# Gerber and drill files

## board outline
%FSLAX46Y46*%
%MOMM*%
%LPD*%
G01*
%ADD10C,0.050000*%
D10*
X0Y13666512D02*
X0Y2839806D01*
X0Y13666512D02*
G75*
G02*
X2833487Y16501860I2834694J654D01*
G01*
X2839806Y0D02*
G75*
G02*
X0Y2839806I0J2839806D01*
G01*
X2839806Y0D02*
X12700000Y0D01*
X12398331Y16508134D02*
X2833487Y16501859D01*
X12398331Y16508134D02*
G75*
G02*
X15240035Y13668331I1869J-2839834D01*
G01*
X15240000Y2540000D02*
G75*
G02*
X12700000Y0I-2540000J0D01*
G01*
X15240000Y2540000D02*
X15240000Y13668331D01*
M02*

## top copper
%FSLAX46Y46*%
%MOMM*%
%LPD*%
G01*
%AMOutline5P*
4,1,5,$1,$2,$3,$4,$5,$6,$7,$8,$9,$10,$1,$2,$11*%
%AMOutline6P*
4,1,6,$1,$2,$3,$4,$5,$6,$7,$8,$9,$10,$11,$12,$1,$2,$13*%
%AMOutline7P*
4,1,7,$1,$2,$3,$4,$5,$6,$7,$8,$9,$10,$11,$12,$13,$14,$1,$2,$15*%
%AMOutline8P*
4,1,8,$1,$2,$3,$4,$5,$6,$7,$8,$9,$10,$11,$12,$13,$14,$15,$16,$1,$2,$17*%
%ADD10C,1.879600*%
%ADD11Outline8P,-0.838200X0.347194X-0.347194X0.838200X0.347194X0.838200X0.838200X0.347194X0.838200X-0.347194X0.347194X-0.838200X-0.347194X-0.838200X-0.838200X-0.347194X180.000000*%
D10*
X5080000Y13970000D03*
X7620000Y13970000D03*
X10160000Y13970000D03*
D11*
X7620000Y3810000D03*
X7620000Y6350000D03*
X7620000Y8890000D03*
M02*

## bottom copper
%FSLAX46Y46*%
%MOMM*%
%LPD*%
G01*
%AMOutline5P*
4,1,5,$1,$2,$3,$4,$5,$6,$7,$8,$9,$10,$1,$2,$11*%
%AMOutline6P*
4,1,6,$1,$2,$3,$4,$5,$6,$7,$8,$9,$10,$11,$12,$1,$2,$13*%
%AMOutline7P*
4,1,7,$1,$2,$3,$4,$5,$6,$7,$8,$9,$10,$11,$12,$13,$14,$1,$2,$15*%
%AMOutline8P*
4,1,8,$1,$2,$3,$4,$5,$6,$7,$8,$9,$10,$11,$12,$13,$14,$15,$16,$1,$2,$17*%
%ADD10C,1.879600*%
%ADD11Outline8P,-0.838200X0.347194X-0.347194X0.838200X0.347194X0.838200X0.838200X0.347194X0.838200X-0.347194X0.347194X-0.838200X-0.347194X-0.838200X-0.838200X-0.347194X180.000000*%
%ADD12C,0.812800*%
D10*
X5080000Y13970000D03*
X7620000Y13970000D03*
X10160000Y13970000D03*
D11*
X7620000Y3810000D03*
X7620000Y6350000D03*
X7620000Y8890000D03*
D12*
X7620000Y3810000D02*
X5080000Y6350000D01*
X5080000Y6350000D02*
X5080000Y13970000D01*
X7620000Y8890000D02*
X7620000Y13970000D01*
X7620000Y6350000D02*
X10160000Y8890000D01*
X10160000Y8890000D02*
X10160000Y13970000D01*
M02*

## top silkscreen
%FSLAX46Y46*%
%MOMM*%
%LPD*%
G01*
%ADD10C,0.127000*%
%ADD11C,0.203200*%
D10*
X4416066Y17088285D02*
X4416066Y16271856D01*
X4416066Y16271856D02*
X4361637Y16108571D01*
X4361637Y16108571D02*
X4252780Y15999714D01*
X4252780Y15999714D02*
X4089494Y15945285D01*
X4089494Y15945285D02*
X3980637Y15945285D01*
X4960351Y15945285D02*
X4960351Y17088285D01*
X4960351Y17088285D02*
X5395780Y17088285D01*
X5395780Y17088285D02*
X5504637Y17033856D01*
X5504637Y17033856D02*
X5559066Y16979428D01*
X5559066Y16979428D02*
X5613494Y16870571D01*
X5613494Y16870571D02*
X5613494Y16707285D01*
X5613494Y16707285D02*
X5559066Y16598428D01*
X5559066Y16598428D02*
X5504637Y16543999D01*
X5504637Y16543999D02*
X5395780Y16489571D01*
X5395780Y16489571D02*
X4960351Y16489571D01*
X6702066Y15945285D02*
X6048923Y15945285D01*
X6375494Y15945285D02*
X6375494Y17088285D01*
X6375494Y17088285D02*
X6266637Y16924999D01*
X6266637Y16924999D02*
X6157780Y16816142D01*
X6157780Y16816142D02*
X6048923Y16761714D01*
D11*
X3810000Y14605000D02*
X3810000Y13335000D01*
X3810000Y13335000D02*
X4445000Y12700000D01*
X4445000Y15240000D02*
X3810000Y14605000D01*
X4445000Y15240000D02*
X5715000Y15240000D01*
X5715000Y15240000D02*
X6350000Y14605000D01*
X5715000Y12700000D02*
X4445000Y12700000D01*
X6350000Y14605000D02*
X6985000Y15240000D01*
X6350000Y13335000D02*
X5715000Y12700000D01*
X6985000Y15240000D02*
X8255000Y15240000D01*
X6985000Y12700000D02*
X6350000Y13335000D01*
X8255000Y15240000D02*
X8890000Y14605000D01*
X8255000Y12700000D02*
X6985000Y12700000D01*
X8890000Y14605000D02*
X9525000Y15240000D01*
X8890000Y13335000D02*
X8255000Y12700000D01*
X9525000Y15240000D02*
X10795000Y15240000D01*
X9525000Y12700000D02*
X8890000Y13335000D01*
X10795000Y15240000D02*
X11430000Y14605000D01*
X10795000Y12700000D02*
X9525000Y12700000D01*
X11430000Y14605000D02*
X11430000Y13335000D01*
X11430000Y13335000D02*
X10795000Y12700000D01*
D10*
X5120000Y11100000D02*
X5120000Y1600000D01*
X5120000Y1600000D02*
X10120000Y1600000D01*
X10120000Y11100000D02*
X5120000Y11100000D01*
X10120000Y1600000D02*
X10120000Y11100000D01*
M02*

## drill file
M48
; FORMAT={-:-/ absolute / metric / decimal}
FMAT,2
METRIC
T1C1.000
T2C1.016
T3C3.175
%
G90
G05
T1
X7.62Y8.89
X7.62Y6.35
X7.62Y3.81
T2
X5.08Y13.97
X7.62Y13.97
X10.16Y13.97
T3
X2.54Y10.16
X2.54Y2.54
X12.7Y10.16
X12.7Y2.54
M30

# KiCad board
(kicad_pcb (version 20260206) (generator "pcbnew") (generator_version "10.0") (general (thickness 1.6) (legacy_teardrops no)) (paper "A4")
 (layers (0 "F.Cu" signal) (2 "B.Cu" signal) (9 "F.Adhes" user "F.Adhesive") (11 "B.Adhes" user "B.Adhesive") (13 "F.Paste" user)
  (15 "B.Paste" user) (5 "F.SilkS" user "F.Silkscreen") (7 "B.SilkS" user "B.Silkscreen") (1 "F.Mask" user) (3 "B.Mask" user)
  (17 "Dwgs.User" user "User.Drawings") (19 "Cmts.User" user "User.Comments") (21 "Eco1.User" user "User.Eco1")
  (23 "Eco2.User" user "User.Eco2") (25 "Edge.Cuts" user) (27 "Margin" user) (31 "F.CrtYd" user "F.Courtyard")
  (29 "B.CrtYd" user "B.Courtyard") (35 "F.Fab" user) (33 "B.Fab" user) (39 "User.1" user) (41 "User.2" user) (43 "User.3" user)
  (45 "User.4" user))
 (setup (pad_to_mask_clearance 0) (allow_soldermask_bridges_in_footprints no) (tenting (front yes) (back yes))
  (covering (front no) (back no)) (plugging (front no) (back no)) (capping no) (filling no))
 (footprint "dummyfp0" (layer "F.Cu") (at 2.54 -2.54)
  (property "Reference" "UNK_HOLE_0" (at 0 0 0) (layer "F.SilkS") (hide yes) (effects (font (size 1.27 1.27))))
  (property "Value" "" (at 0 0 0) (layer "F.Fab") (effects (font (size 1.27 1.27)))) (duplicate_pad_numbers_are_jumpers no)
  (pad "" np_thru_hole circle (at 0 0) (size 3.175 3.175) (drill 3.175) (layers "*.Cu" "*.Mask")))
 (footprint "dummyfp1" (layer "F.Cu") (at 2.54 -10.16)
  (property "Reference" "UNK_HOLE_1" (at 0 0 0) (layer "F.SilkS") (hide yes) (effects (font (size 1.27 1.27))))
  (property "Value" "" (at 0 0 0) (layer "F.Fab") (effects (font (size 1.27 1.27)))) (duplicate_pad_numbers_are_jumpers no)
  (pad "" np_thru_hole circle (at 0 0) (size 3.175 3.175) (drill 3.175) (layers "*.Cu" "*.Mask")))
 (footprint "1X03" (layer "F.Cu") (at 5.08 -13.97)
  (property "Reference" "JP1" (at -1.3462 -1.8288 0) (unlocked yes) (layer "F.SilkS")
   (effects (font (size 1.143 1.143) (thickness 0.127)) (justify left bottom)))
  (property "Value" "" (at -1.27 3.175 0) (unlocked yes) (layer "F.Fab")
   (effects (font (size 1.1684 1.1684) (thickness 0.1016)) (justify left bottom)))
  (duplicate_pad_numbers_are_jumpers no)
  (fp_line (start -1.27 -0.635) (end -1.27 0.635) (stroke (width 0.2032) (type solid)) (layer "F.SilkS"))
  (fp_line (start -1.27 0.635) (end -0.635 1.27) (stroke (width 0.2032) (type solid)) (layer "F.SilkS"))
  (fp_line (start -0.635 -1.27) (end -1.27 -0.635) (stroke (width 0.2032) (type solid)) (layer "F.SilkS"))
  (fp_line (start -0.635 -1.27) (end 0.635 -1.27) (stroke (width 0.2032) (type solid)) (layer "F.SilkS"))
  (fp_line (start 0.635 -1.27) (end 1.27 -0.635) (stroke (width 0.2032) (type solid)) (layer "F.SilkS"))
  (fp_line (start 0.635 1.27) (end -0.635 1.27) (stroke (width 0.2032) (type solid)) (layer "F.SilkS"))
  (fp_line (start 1.27 -0.635) (end 1.905 -1.27) (stroke (width 0.2032) (type solid)) (layer "F.SilkS"))
  (fp_line (start 1.27 0.635) (end 0.635 1.27) (stroke (width 0.2032) (type solid)) (layer "F.SilkS"))
  (fp_line (start 1.905 -1.27) (end 3.175 -1.27) (stroke (width 0.2032) (type solid)) (layer "F.SilkS"))
  (fp_line (start 1.905 1.27) (end 1.27 0.635) (stroke (width 0.2032) (type solid)) (layer "F.SilkS"))
  (fp_line (start 3.175 -1.27) (end 3.81 -0.635) (stroke (width 0.2032) (type solid)) (layer "F.SilkS"))
  (fp_line (start 3.175 1.27) (end 1.905 1.27) (stroke (width 0.2032) (type solid)) (layer "F.SilkS"))
  (fp_line (start 3.81 -0.635) (end 4.445 -1.27) (stroke (width 0.2032) (type solid)) (layer "F.SilkS"))
  (fp_line (start 3.81 0.635) (end 3.175 1.27) (stroke (width 0.2032) (type solid)) (layer "F.SilkS"))
  (fp_line (start 4.445 -1.27) (end 5.715 -1.27) (stroke (width 0.2032) (type solid)) (layer "F.SilkS"))
  (fp_line (start 4.445 1.27) (end 3.81 0.635) (stroke (width 0.2032) (type solid)) (layer "F.SilkS"))
  (fp_line (start 5.715 -1.27) (end 6.35 -0.635) (stroke (width 0.2032) (type solid)) (layer "F.SilkS"))
  (fp_line (start 5.715 1.27) (end 4.445 1.27) (stroke (width 0.2032) (type solid)) (layer "F.SilkS"))
  (fp_line (start 6.35 -0.635) (end 6.35 0.635) (stroke (width 0.2032) (type solid)) (layer "F.SilkS"))
  (fp_line (start 6.35 0.635) (end 5.715 1.27) (stroke (width 0.2032) (type solid)) (layer "F.SilkS"))
  (pad "1" thru_hole circle (at 0 0 90) (size 1.8796 1.8796) (drill 1.016) (layers "*.Cu" "*.Mask") (remove_unused_layers no) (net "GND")
   (solder_mask_margin 0.1016) (thermal_bridge_angle 0))
  (pad "2" thru_hole circle (at 2.54 0 90) (size 1.8796 1.8796) (drill 1.016) (layers "*.Cu" "*.Mask") (remove_unused_layers no) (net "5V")
   (solder_mask_margin 0.1016) (thermal_bridge_angle 0))
  (pad "3" thru_hole circle (at 5.08 0 90) (size 1.8796 1.8796) (drill 1.016) (layers "*.Cu" "*.Mask") (remove_unused_layers no) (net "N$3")
   (solder_mask_margin 0.1016) (thermal_bridge_angle 0)))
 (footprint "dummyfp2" (layer "F.Cu") (at 12.7 -10.16)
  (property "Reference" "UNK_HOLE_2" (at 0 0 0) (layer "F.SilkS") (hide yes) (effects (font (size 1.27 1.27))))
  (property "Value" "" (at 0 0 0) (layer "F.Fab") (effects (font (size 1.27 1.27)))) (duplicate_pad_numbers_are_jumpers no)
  (pad "" np_thru_hole circle (at 0 0) (size 3.175 3.175) (drill 3.175) (layers "*.Cu" "*.Mask")))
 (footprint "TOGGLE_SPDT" (layer "F.Cu") (at 7.62 -6.35 180)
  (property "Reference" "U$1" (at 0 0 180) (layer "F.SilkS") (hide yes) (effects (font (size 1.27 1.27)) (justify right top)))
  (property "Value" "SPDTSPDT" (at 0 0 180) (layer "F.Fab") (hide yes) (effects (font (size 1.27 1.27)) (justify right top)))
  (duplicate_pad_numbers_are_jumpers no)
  (fp_line (start 2.5 4.75) (end 2.5 -4.75) (stroke (width 0.127) (type solid)) (layer "F.SilkS"))
  (fp_line (start 2.5 -4.75) (end -2.5 -4.75) (stroke (width 0.127) (type solid)) (layer "F.SilkS"))
  (fp_line (start -2.5 4.75) (end 2.5 4.75) (stroke (width 0.127) (type solid)) (layer "F.SilkS"))
  (fp_line (start -2.5 -4.75) (end -2.5 4.75) (stroke (width 0.127) (type solid)) (layer "F.SilkS"))
  (pad "1" thru_hole roundrect (at 0 -2.54 180) (size 1.6764 1.6764) (drill 1) (layers "*.Cu" "*.Mask") (remove_unused_layers no)
   (roundrect_rratio 0.25) (chamfer_ratio 0.2928932188) (chamfer top_left top_right bottom_left bottom_right) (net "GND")
   (solder_mask_margin 0.1016) (thermal_bridge_angle 0))
  (pad "2" thru_hole roundrect (at 0 0 180) (size 1.6764 1.6764) (drill 1) (layers "*.Cu" "*.Mask") (remove_unused_layers no)
   (roundrect_rratio 0.25) (chamfer_ratio 0.2928932188) (chamfer top_left top_right bottom_left bottom_right) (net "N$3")
   (solder_mask_margin 0.1016) (thermal_bridge_angle 0))
  (pad "3" thru_hole roundrect (at 0 2.54 180) (size 1.6764 1.6764) (drill 1) (layers "*.Cu" "*.Mask") (remove_unused_layers no)
   (roundrect_rratio 0.25) (chamfer_ratio 0.2928932188) (chamfer top_left top_right bottom_left bottom_right) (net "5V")
   (solder_mask_margin 0.1016) (thermal_bridge_angle 0)))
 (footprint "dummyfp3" (layer "F.Cu") (at 12.7 -2.54)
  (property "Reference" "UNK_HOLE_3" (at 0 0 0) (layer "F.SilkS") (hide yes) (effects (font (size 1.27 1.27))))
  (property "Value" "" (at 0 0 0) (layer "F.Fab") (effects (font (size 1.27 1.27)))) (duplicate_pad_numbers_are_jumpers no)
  (pad "" np_thru_hole circle (at 0 0) (size 3.175 3.175) (drill 3.175) (layers "*.Cu" "*.Mask")))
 (gr_line (start 0 -13.666512) (end 0 -2.839806) (stroke (width 0.05) (type solid)) (layer "Edge.Cuts"))
 (gr_arc (start 0 -13.666512) (mid 0.829605 -15.670939) (end 2.833487 -16.501859) (stroke (width 0.05) (type solid)) (layer "Edge.Cuts"))
 (gr_arc (start 2.839806 0) (mid 0.83176 -0.83176) (end 0 -2.839806) (stroke (width 0.05) (type solid)) (layer "Edge.Cuts"))
 (gr_line (start 2.839806 0) (end 12.7 0) (stroke (width 0.05) (type solid)) (layer "Edge.Cuts"))
 (gr_line (start 12.398331 -16.508134) (end 2.833487 -16.501859) (stroke (width 0.05) (type solid)) (layer "Edge.Cuts"))
 (gr_arc (start 12.398331 -16.508134) (mid 14.407581 -15.677034) (end 15.24 -13.668331) (stroke (width 0.05) (type solid))
  (layer "Edge.Cuts"))
 (gr_arc (start 15.24 -2.54) (mid 14.496051 -0.743949) (end 12.7 0) (stroke (width 0.05) (type solid)) (layer "Edge.Cuts"))
 (gr_line (start 15.24 -2.54) (end 15.24 -13.668331) (stroke (width 0.05) (type solid)) (layer "Edge.Cuts"))
 (segment (start 7.62 -3.81) (end 5.08 -6.35) (width 0.8128) (layer "B.Cu") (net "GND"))
 (segment (start 5.08 -6.35) (end 5.08 -13.97) (width 0.8128) (layer "B.Cu") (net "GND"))
 (segment (start 7.62 -8.89) (end 7.62 -13.97) (width 0.8128) (layer "B.Cu") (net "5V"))
 (segment (start 7.62 -6.35) (end 10.16 -8.89) (width 0.8128) (layer "B.Cu") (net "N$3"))
 (segment (start 10.16 -8.89) (end 10.16 -13.97) (width 0.8128) (layer "B.Cu") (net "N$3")))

